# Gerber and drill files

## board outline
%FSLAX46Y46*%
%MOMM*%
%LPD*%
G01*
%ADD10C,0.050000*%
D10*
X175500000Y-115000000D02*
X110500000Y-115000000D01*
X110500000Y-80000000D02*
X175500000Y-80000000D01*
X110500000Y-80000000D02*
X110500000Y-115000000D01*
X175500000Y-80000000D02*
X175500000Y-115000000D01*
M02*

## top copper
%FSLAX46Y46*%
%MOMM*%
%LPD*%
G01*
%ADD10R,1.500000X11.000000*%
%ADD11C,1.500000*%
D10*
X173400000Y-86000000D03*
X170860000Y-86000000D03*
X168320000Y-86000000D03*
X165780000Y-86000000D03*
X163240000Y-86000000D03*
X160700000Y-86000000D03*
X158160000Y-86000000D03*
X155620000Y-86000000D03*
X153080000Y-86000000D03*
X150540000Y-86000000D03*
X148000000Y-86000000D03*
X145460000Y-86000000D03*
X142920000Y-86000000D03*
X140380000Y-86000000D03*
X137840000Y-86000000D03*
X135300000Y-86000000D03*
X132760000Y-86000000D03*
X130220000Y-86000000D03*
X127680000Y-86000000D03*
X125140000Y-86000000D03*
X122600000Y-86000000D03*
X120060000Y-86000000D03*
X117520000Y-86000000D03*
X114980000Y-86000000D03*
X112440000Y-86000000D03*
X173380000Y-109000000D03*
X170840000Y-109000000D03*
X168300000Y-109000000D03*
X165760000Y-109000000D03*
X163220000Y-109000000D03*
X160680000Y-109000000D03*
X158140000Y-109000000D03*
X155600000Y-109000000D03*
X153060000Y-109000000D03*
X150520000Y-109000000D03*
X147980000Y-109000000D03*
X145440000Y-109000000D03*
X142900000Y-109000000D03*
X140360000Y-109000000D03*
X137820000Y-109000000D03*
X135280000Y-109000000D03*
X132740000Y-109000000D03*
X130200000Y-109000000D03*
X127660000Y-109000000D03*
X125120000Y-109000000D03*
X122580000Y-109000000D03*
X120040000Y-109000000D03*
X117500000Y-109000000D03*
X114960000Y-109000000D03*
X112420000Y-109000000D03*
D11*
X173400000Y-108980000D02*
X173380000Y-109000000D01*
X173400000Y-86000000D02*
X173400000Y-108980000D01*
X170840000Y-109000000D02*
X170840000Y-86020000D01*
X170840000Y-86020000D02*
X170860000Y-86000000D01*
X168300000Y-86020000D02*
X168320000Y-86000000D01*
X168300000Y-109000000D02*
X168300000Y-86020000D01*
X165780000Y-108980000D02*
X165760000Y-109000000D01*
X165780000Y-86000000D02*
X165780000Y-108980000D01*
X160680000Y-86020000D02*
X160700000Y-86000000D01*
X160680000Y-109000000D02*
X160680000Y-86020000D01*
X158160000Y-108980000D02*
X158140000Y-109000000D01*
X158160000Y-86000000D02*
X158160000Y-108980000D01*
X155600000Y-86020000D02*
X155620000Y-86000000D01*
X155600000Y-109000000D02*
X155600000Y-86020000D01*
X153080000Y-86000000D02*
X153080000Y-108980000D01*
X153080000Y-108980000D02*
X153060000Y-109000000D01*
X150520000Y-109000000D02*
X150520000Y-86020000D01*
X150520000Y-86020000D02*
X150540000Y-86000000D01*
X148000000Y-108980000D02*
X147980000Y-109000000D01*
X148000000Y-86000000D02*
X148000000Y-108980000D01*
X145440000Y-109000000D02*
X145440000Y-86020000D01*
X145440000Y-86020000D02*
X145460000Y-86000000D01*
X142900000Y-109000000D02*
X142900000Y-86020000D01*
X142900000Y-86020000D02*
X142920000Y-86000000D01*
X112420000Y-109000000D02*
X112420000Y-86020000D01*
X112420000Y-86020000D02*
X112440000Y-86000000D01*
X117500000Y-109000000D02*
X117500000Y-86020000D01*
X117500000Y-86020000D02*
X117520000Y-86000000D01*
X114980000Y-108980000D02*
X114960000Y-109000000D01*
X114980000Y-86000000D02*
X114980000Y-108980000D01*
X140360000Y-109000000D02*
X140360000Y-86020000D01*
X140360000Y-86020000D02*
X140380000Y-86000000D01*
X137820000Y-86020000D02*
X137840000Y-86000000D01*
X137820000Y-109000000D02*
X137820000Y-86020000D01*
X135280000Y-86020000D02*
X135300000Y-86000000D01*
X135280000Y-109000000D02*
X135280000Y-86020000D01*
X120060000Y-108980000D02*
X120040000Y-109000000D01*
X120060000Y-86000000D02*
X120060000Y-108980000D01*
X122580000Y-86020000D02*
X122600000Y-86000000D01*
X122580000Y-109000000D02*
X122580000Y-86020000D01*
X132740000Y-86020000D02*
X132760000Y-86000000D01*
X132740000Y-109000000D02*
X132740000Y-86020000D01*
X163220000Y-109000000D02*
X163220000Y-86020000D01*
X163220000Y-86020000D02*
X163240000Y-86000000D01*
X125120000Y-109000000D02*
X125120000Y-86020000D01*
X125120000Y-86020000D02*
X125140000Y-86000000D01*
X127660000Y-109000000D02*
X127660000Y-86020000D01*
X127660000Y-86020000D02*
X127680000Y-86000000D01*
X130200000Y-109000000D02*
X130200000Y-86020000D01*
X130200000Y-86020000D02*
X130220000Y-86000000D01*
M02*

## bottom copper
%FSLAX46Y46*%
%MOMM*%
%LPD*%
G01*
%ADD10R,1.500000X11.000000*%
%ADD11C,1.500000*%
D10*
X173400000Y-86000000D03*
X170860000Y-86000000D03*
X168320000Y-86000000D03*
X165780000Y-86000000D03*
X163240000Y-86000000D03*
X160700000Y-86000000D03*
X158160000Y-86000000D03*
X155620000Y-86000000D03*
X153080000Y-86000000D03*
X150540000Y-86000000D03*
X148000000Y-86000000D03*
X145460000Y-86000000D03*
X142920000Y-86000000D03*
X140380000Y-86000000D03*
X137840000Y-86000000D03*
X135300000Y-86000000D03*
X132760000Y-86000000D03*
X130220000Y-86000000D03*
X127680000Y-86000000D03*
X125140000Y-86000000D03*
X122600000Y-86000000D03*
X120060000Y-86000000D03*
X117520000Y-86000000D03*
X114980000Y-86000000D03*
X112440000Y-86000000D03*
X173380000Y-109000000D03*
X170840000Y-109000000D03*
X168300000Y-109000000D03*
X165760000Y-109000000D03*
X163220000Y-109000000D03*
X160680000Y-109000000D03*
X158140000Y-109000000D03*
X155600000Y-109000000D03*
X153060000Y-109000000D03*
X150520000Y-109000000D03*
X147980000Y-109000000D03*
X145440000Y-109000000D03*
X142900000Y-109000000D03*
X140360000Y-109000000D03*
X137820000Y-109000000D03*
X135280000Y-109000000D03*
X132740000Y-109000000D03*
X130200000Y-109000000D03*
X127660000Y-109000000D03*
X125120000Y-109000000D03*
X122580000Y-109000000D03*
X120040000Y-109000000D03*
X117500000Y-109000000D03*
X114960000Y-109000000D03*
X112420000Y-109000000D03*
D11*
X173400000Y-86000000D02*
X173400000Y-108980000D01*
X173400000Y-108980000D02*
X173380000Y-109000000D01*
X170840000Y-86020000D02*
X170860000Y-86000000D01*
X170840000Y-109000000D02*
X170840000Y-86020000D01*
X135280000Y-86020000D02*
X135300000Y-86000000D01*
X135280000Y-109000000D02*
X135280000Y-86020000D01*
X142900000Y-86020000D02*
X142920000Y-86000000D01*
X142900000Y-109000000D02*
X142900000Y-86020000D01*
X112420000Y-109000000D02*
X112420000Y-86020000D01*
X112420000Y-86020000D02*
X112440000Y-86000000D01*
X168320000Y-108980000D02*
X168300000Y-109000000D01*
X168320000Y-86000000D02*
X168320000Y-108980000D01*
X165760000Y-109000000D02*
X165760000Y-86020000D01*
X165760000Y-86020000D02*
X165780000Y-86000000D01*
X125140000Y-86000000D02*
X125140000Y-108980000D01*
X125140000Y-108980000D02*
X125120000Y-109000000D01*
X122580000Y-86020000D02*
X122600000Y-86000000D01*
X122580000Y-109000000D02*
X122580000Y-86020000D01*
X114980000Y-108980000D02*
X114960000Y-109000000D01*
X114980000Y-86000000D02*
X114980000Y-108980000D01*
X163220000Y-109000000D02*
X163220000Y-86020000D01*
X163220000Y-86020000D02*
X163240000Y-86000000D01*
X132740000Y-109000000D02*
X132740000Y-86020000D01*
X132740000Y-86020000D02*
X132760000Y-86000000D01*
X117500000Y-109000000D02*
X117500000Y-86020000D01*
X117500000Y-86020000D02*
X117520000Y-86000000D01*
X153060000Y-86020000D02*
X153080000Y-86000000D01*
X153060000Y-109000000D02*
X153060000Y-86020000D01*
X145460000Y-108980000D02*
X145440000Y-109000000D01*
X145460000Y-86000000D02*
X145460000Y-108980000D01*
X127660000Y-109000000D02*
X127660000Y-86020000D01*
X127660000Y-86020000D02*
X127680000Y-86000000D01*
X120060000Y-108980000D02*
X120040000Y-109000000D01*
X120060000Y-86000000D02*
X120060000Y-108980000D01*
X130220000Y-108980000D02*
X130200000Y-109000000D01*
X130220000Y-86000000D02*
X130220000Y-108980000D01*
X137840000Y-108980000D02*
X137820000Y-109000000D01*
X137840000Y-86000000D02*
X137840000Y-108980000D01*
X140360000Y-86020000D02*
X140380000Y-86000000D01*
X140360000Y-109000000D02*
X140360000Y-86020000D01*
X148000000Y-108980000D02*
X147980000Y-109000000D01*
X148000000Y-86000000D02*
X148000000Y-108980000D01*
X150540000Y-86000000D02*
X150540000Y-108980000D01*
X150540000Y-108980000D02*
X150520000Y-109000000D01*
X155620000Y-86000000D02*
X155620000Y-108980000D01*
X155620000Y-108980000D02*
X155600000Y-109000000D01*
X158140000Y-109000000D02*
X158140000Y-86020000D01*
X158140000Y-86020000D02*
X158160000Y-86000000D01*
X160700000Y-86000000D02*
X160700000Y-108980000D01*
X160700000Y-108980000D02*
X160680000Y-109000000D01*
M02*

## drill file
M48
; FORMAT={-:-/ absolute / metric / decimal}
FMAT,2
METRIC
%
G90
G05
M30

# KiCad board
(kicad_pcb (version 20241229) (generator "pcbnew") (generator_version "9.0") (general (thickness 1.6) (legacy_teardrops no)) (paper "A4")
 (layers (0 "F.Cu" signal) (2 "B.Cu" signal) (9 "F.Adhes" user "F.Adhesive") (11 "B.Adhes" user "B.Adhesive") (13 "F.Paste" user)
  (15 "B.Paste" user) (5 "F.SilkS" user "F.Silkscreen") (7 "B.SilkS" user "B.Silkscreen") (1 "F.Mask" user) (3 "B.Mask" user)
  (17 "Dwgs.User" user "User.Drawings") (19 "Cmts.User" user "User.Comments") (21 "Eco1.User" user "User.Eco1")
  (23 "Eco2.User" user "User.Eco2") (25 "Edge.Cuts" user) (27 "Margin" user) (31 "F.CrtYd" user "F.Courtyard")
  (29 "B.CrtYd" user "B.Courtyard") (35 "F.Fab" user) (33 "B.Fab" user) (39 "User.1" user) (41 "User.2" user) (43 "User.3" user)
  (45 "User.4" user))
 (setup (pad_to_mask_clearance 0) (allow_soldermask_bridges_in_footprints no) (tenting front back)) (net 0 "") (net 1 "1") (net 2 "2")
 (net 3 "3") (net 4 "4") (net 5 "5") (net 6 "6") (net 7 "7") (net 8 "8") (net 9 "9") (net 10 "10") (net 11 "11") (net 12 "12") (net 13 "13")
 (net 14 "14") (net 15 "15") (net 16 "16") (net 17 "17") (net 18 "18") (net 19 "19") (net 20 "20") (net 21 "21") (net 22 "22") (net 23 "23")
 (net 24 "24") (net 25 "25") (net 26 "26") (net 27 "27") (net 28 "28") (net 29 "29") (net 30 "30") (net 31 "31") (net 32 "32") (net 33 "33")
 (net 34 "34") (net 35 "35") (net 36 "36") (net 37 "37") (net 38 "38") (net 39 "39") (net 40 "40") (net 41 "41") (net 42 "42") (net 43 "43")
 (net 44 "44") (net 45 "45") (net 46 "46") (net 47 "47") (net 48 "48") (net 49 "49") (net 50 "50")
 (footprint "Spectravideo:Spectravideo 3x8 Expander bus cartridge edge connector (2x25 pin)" (layer "F.Cu") (at 143 86)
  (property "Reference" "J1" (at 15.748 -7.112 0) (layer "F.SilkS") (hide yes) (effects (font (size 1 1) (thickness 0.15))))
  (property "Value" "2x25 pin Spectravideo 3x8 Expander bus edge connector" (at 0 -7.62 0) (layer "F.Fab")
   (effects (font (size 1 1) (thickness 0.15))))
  (pad "1" connect rect (at 30.4 0) (size 1.5 11) (layers "F.Cu" "F.Mask") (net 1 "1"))
  (pad "2" connect rect (at 30.4 0) (size 1.5 11) (layers "B.Cu" "B.Mask") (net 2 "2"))
  (pad "3" connect rect (at 27.86 0) (size 1.5 11) (layers "F.Cu" "F.Mask") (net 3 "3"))
  (pad "4" connect rect (at 27.86 0) (size 1.5 11) (layers "B.Cu" "B.Mask") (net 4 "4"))
  (pad "5" connect rect (at 25.32 0) (size 1.5 11) (layers "F.Cu" "F.Mask") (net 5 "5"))
  (pad "6" connect rect (at 25.32 0) (size 1.5 11) (layers "B.Cu" "B.Mask") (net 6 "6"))
  (pad "7" connect rect (at 22.78 0) (size 1.5 11) (layers "F.Cu" "F.Mask") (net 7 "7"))
  (pad "8" connect rect (at 22.78 0) (size 1.5 11) (layers "B.Cu" "B.Mask") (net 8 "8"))
  (pad "9" connect rect (at 20.24 0) (size 1.5 11) (layers "F.Cu" "F.Mask") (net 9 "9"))
  (pad "10" connect rect (at 20.24 0) (size 1.5 11) (layers "B.Cu" "B.Mask") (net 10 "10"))
  (pad "11" connect rect (at 17.7 0) (size 1.5 11) (layers "F.Cu" "F.Mask") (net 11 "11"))
  (pad "12" connect rect (at 17.7 0) (size 1.5 11) (layers "B.Cu" "B.Mask") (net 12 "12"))
  (pad "13" connect rect (at 15.16 0) (size 1.5 11) (layers "F.Cu" "F.Mask") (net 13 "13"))
  (pad "14" connect rect (at 15.16 0) (size 1.5 11) (layers "B.Cu" "B.Mask") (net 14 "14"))
  (pad "15" connect rect (at 12.62 0) (size 1.5 11) (layers "F.Cu" "F.Mask") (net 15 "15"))
  (pad "16" connect rect (at 12.62 0) (size 1.5 11) (layers "B.Cu" "B.Mask") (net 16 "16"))
  (pad "17" connect rect (at 10.08 0) (size 1.5 11) (layers "F.Cu" "F.Mask") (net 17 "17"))
  (pad "18" connect rect (at 10.08 0) (size 1.5 11) (layers "B.Cu" "B.Mask") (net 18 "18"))
  (pad "19" connect rect (at 7.54 0) (size 1.5 11) (layers "F.Cu" "F.Mask") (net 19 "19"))
  (pad "20" connect rect (at 7.54 0) (size 1.5 11) (layers "B.Cu" "B.Mask") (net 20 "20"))
  (pad "21" connect rect (at 5 0) (size 1.5 11) (layers "F.Cu" "F.Mask") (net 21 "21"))
  (pad "22" connect rect (at 5 0) (size 1.5 11) (layers "B.Cu" "B.Mask") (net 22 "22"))
  (pad "23" connect rect (at 2.46 0) (size 1.5 11) (layers "F.Cu" "F.Mask") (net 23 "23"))
  (pad "24" connect rect (at 2.46 0) (size 1.5 11) (layers "B.Cu" "B.Mask") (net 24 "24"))
  (pad "25" connect rect (at -0.08 0) (size 1.5 11) (layers "F.Cu" "F.Mask") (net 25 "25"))
  (pad "26" connect rect (at -0.08 0) (size 1.5 11) (layers "B.Cu" "B.Mask") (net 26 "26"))
  (pad "27" connect rect (at -2.62 0) (size 1.5 11) (layers "F.Cu" "F.Mask") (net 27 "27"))
  (pad "28" connect rect (at -2.62 0) (size 1.5 11) (layers "B.Cu" "B.Mask") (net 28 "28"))
  (pad "29" connect rect (at -5.16 0) (size 1.5 11) (layers "F.Cu" "F.Mask") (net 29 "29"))
  (pad "30" connect rect (at -5.16 0) (size 1.5 11) (layers "B.Cu" "B.Mask") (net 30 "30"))
  (pad "31" connect rect (at -7.7 0) (size 1.5 11) (layers "F.Cu" "F.Mask") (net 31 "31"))
  (pad "32" connect rect (at -7.7 0) (size 1.5 11) (layers "B.Cu" "B.Mask") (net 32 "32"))
  (pad "33" connect rect (at -10.24 0) (size 1.5 11) (layers "F.Cu" "F.Mask") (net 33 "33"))
  (pad "34" connect rect (at -10.24 0) (size 1.5 11) (layers "B.Cu" "B.Mask") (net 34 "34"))
  (pad "35" connect rect (at -12.78 0) (size 1.5 11) (layers "F.Cu" "F.Mask") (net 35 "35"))
  (pad "36" connect rect (at -12.78 0) (size 1.5 11) (layers "B.Cu" "B.Mask") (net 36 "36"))
  (pad "37" connect rect (at -15.32 0) (size 1.5 11) (layers "F.Cu" "F.Mask") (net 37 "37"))
  (pad "38" connect rect (at -15.32 0) (size 1.5 11) (layers "B.Cu" "B.Mask") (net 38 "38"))
  (pad "39" connect rect (at -17.86 0) (size 1.5 11) (layers "F.Cu" "F.Mask") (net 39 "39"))
  (pad "40" connect rect (at -17.86 0) (size 1.5 11) (layers "B.Cu" "B.Mask") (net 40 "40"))
  (pad "41" connect rect (at -20.4 0) (size 1.5 11) (layers "F.Cu" "F.Mask") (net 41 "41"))
  (pad "42" connect rect (at -20.4 0) (size 1.5 11) (layers "B.Cu" "B.Mask") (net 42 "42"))
  (pad "43" connect rect (at -22.94 0) (size 1.5 11) (layers "F.Cu" "F.Mask") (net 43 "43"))
  (pad "44" connect rect (at -22.94 0) (size 1.5 11) (layers "B.Cu" "B.Mask") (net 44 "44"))
  (pad "45" connect rect (at -25.48 0) (size 1.5 11) (layers "F.Cu" "F.Mask") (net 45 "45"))
  (pad "46" connect rect (at -25.48 0) (size 1.5 11) (layers "B.Cu" "B.Mask") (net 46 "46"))
  (pad "47" connect rect (at -28.02 0) (size 1.5 11) (layers "F.Cu" "F.Mask") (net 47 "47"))
  (pad "48" connect rect (at -28.02 0) (size 1.5 11) (layers "B.Cu" "B.Mask") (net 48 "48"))
  (pad "49" connect rect (at -30.56 0) (size 1.5 11) (layers "F.Cu" "F.Mask") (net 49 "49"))
  (pad "50" connect rect (at -30.56 0) (size 1.5 11) (layers "B.Cu" "B.Mask") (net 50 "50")))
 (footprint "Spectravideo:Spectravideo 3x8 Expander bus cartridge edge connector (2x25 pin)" (layer "F.Cu") (at 142.98 109)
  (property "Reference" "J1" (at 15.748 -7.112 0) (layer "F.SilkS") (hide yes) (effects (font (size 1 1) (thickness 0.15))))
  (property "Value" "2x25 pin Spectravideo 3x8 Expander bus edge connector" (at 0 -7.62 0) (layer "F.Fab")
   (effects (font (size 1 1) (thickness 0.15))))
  (pad "1" connect rect (at 30.4 0) (size 1.5 11) (layers "F.Cu" "F.Mask") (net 1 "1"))
  (pad "2" connect rect (at 30.4 0) (size 1.5 11) (layers "B.Cu" "B.Mask") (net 2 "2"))
  (pad "3" connect rect (at 27.86 0) (size 1.5 11) (layers "F.Cu" "F.Mask") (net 3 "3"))
  (pad "4" connect rect (at 27.86 0) (size 1.5 11) (layers "B.Cu" "B.Mask") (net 4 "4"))
  (pad "5" connect rect (at 25.32 0) (size 1.5 11) (layers "F.Cu" "F.Mask") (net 5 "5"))
  (pad "6" connect rect (at 25.32 0) (size 1.5 11) (layers "B.Cu" "B.Mask") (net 6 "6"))
  (pad "7" connect rect (at 22.78 0) (size 1.5 11) (layers "F.Cu" "F.Mask") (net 7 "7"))
  (pad "8" connect rect (at 22.78 0) (size 1.5 11) (layers "B.Cu" "B.Mask") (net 8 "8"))
  (pad "9" connect rect (at 20.24 0) (size 1.5 11) (layers "F.Cu" "F.Mask") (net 9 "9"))
  (pad "10" connect rect (at 20.24 0) (size 1.5 11) (layers "B.Cu" "B.Mask") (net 10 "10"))
  (pad "11" connect rect (at 17.7 0) (size 1.5 11) (layers "F.Cu" "F.Mask") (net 11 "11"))
  (pad "12" connect rect (at 17.7 0) (size 1.5 11) (layers "B.Cu" "B.Mask") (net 12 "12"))
  (pad "13" connect rect (at 15.16 0) (size 1.5 11) (layers "F.Cu" "F.Mask") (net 13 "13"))
  (pad "14" connect rect (at 15.16 0) (size 1.5 11) (layers "B.Cu" "B.Mask") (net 14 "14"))
  (pad "15" connect rect (at 12.62 0) (size 1.5 11) (layers "F.Cu" "F.Mask") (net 15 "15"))
  (pad "16" connect rect (at 12.62 0) (size 1.5 11) (layers "B.Cu" "B.Mask") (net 16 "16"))
  (pad "17" connect rect (at 10.08 0) (size 1.5 11) (layers "F.Cu" "F.Mask") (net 17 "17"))
  (pad "18" connect rect (at 10.08 0) (size 1.5 11) (layers "B.Cu" "B.Mask") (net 18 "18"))
  (pad "19" connect rect (at 7.54 0) (size 1.5 11) (layers "F.Cu" "F.Mask") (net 19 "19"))
  (pad "20" connect rect (at 7.54 0) (size 1.5 11) (layers "B.Cu" "B.Mask") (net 20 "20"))
  (pad "21" connect rect (at 5 0) (size 1.5 11) (layers "F.Cu" "F.Mask") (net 21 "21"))
  (pad "22" connect rect (at 5 0) (size 1.5 11) (layers "B.Cu" "B.Mask") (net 22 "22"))
  (pad "23" connect rect (at 2.46 0) (size 1.5 11) (layers "F.Cu" "F.Mask") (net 23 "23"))
  (pad "24" connect rect (at 2.46 0) (size 1.5 11) (layers "B.Cu" "B.Mask") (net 24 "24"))
  (pad "25" connect rect (at -0.08 0) (size 1.5 11) (layers "F.Cu" "F.Mask") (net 25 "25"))
  (pad "26" connect rect (at -0.08 0) (size 1.5 11) (layers "B.Cu" "B.Mask") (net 26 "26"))
  (pad "27" connect rect (at -2.62 0) (size 1.5 11) (layers "F.Cu" "F.Mask") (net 27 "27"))
  (pad "28" connect rect (at -2.62 0) (size 1.5 11) (layers "B.Cu" "B.Mask") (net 28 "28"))
  (pad "29" connect rect (at -5.16 0) (size 1.5 11) (layers "F.Cu" "F.Mask") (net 29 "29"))
  (pad "30" connect rect (at -5.16 0) (size 1.5 11) (layers "B.Cu" "B.Mask") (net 30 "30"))
  (pad "31" connect rect (at -7.7 0) (size 1.5 11) (layers "F.Cu" "F.Mask") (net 31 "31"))
  (pad "32" connect rect (at -7.7 0) (size 1.5 11) (layers "B.Cu" "B.Mask") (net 32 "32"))
  (pad "33" connect rect (at -10.24 0) (size 1.5 11) (layers "F.Cu" "F.Mask") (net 33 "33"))
  (pad "34" connect rect (at -10.24 0) (size 1.5 11) (layers "B.Cu" "B.Mask") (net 34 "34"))
  (pad "35" connect rect (at -12.78 0) (size 1.5 11) (layers "F.Cu" "F.Mask") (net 35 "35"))
  (pad "36" connect rect (at -12.78 0) (size 1.5 11) (layers "B.Cu" "B.Mask") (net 36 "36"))
  (pad "37" connect rect (at -15.32 0) (size 1.5 11) (layers "F.Cu" "F.Mask") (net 37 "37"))
  (pad "38" connect rect (at -15.32 0) (size 1.5 11) (layers "B.Cu" "B.Mask") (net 38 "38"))
  (pad "39" connect rect (at -17.86 0) (size 1.5 11) (layers "F.Cu" "F.Mask") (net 39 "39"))
  (pad "40" connect rect (at -17.86 0) (size 1.5 11) (layers "B.Cu" "B.Mask") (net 40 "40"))
  (pad "41" connect rect (at -20.4 0) (size 1.5 11) (layers "F.Cu" "F.Mask") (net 41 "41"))
  (pad "42" connect rect (at -20.4 0) (size 1.5 11) (layers "B.Cu" "B.Mask") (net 42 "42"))
  (pad "43" connect rect (at -22.94 0) (size 1.5 11) (layers "F.Cu" "F.Mask") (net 43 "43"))
  (pad "44" connect rect (at -22.94 0) (size 1.5 11) (layers "B.Cu" "B.Mask") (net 44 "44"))
  (pad "45" connect rect (at -25.48 0) (size 1.5 11) (layers "F.Cu" "F.Mask") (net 45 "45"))
  (pad "46" connect rect (at -25.48 0) (size 1.5 11) (layers "B.Cu" "B.Mask") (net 46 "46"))
  (pad "47" connect rect (at -28.02 0) (size 1.5 11) (layers "F.Cu" "F.Mask") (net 47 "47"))
  (pad "48" connect rect (at -28.02 0) (size 1.5 11) (layers "B.Cu" "B.Mask") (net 48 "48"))
  (pad "49" connect rect (at -30.56 0) (size 1.5 11) (layers "F.Cu" "F.Mask") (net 49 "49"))
  (pad "50" connect rect (at -30.56 0) (size 1.5 11) (layers "B.Cu" "B.Mask") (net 50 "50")))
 (gr_line (start 175.5 115) (end 110.5 115) (stroke (width 0.05) (type default)) (layer "Edge.Cuts"))
 (gr_line (start 110.5 80) (end 175.5 80) (stroke (width 0.05) (type default)) (layer "Edge.Cuts"))
 (gr_line (start 110.5 80) (end 110.5 115) (stroke (width 0.05) (type default)) (layer "Edge.Cuts"))
 (gr_line (start 175.5 80) (end 175.5 115) (stroke (width 0.05) (type default)) (layer "Edge.Cuts"))
 (segment (start 173.4 108.98) (end 173.38 109) (width 1.5) (layer "F.Cu") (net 1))
 (segment (start 173.4 86) (end 173.4 108.98) (width 1.5) (layer "F.Cu") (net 1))
 (segment (start 170.84 109) (end 170.84 86.02) (width 1.5) (layer "F.Cu") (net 3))
 (segment (start 170.84 86.02) (end 170.86 86) (width 1.5) (layer "F.Cu") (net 3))
 (segment (start 168.3 86.02) (end 168.32 86) (width 1.5) (layer "F.Cu") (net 5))
 (segment (start 168.3 109) (end 168.3 86.02) (width 1.5) (layer "F.Cu") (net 5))
 (segment (start 165.78 108.98) (end 165.76 109) (width 1.5) (layer "F.Cu") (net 7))
 (segment (start 165.78 86) (end 165.78 108.98) (width 1.5) (layer "F.Cu") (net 7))
 (segment (start 160.68 86.02) (end 160.7 86) (width 1.5) (layer "F.Cu") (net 11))
 (segment (start 160.68 109) (end 160.68 86.02) (width 1.5) (layer "F.Cu") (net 11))
 (segment (start 158.16 108.98) (end 158.14 109) (width 1.5) (layer "F.Cu") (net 13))
 (segment (start 158.16 86) (end 158.16 108.98) (width 1.5) (layer "F.Cu") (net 13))
 (segment (start 155.6 86.02) (end 155.62 86) (width 1.5) (layer "F.Cu") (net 15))
 (segment (start 155.6 109) (end 155.6 86.02) (width 1.5) (layer "F.Cu") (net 15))
 (segment (start 153.08 86) (end 153.08 108.98) (width 1.5) (layer "F.Cu") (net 17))
 (segment (start 153.08 108.98) (end 153.06 109) (width 1.5) (layer "F.Cu") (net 17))
 (segment (start 150.52 109) (end 150.52 86.02) (width 1.5) (layer "F.Cu") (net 19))
 (segment (start 150.52 86.02) (end 150.54 86) (width 1.5) (layer "F.Cu") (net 19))
 (segment (start 148 108.98) (end 147.98 109) (width 1.5) (layer "F.Cu") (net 21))
 (segment (start 148 86) (end 148 108.98) (width 1.5) (layer "F.Cu") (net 21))
 (segment (start 145.44 109) (end 145.44 86.02) (width 1.5) (layer "F.Cu") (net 23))
 (segment (start 145.44 86.02) (end 145.46 86) (width 1.5) (layer "F.Cu") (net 23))
 (segment (start 142.9 109) (end 142.9 86.02) (width 1.5) (layer "F.Cu") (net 25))
 (segment (start 142.9 86.02) (end 142.92 86) (width 1.5) (layer "F.Cu") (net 25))
 (segment (start 112.42 109) (end 112.42 86.02) (width 1.5) (layer "F.Cu") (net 49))
 (segment (start 112.42 86.02) (end 112.44 86) (width 1.5) (layer "F.Cu") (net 49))
 (segment (start 117.5 109) (end 117.5 86.02) (width 1.5) (layer "F.Cu") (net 45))
 (segment (start 117.5 86.02) (end 117.52 86) (width 1.5) (layer "F.Cu") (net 45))
 (segment (start 114.98 108.98) (end 114.96 109) (width 1.5) (layer "F.Cu") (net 47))
 (segment (start 114.98 86) (end 114.98 108.98) (width 1.5) (layer "F.Cu") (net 47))
 (segment (start 140.36 109) (end 140.36 86.02) (width 1.5) (layer "F.Cu") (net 27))
 (segment (start 140.36 86.02) (end 140.38 86) (width 1.5) (layer "F.Cu") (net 27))
 (segment (start 137.82 86.02) (end 137.84 86) (width 1.5) (layer "F.Cu") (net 29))
 (segment (start 137.82 109) (end 137.82 86.02) (width 1.5) (layer "F.Cu") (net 29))
 (segment (start 135.28 86.02) (end 135.3 86) (width 1.5) (layer "F.Cu") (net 31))
 (segment (start 135.28 109) (end 135.28 86.02) (width 1.5) (layer "F.Cu") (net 31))
 (segment (start 120.06 108.98) (end 120.04 109) (width 1.5) (layer "F.Cu") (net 43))
 (segment (start 120.06 86) (end 120.06 108.98) (width 1.5) (layer "F.Cu") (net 43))
 (segment (start 122.58 86.02) (end 122.6 86) (width 1.5) (layer "F.Cu") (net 41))
 (segment (start 122.58 109) (end 122.58 86.02) (width 1.5) (layer "F.Cu") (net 41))
 (segment (start 132.74 86.02) (end 132.76 86) (width 1.5) (layer "F.Cu") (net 33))
 (segment (start 132.74 109) (end 132.74 86.02) (width 1.5) (layer "F.Cu") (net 33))
 (segment (start 163.22 109) (end 163.22 86.02) (width 1.5) (layer "F.Cu") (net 9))
 (segment (start 163.22 86.02) (end 163.24 86) (width 1.5) (layer "F.Cu") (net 9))
 (segment (start 125.12 109) (end 125.12 86.02) (width 1.5) (layer "F.Cu") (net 39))
 (segment (start 125.12 86.02) (end 125.14 86) (width 1.5) (layer "F.Cu") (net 39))
 (segment (start 127.66 109) (end 127.66 86.02) (width 1.5) (layer "F.Cu") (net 37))
 (segment (start 127.66 86.02) (end 127.68 86) (width 1.5) (layer "F.Cu") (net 37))
 (segment (start 130.2 109) (end 130.2 86.02) (width 1.5) (layer "F.Cu") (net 35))
 (segment (start 130.2 86.02) (end 130.22 86) (width 1.5) (layer "F.Cu") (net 35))
 (segment (start 173.4 86) (end 173.4 108.98) (width 1.5) (layer "B.Cu") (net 2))
 (segment (start 173.4 108.98) (end 173.38 109) (width 1.5) (layer "B.Cu") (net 2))
 (segment (start 170.84 86.02) (end 170.86 86) (width 1.5) (layer "B.Cu") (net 4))
 (segment (start 170.84 109) (end 170.84 86.02) (width 1.5) (layer "B.Cu") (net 4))
 (segment (start 135.28 86.02) (end 135.3 86) (width 1.5) (layer "B.Cu") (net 32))
 (segment (start 135.28 109) (end 135.28 86.02) (width 1.5) (layer "B.Cu") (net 32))
 (segment (start 142.9 86.02) (end 142.92 86) (width 1.5) (layer "B.Cu") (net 26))
 (segment (start 142.9 109) (end 142.9 86.02) (width 1.5) (layer "B.Cu") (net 26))
 (segment (start 112.42 109) (end 112.42 86.02) (width 1.5) (layer "B.Cu") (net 50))
 (segment (start 112.42 86.02) (end 112.44 86) (width 1.5) (layer "B.Cu") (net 50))
 (segment (start 168.32 108.98) (end 168.3 109) (width 1.5) (layer "B.Cu") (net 6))
 (segment (start 168.32 86) (end 168.32 108.98) (width 1.5) (layer "B.Cu") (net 6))
 (segment (start 165.76 109) (end 165.76 86.02) (width 1.5) (layer "B.Cu") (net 8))
 (segment (start 165.76 86.02) (end 165.78 86) (width 1.5) (layer "B.Cu") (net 8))
 (segment (start 125.14 86) (end 125.14 108.98) (width 1.5) (layer "B.Cu") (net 40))
 (segment (start 125.14 108.98) (end 125.12 109) (width 1.5) (layer "B.Cu") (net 40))
 (segment (start 122.58 86.02) (end 122.6 86) (width 1.5) (layer "B.Cu") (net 42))
 (segment (start 122.58 109) (end 122.58 86.02) (width 1.5) (layer "B.Cu") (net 42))
 (segment (start 114.98 108.98) (end 114.96 109) (width 1.5) (layer "B.Cu") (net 48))
 (segment (start 114.98 86) (end 114.98 108.98) (width 1.5) (layer "B.Cu") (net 48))
 (segment (start 163.22 109) (end 163.22 86.02) (width 1.5) (layer "B.Cu") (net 10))
 (segment (start 163.22 86.02) (end 163.24 86) (width 1.5) (layer "B.Cu") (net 10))
 (segment (start 132.74 109) (end 132.74 86.02) (width 1.5) (layer "B.Cu") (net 34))
 (segment (start 132.74 86.02) (end 132.76 86) (width 1.5) (layer "B.Cu") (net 34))
 (segment (start 117.5 109) (end 117.5 86.02) (width 1.5) (layer "B.Cu") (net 46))
 (segment (start 117.5 86.02) (end 117.52 86) (width 1.5) (layer "B.Cu") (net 46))
 (segment (start 153.06 86.02) (end 153.08 86) (width 1.5) (layer "B.Cu") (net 18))
 (segment (start 153.06 109) (end 153.06 86.02) (width 1.5) (layer "B.Cu") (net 18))
 (segment (start 145.46 108.98) (end 145.44 109) (width 1.5) (layer "B.Cu") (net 24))
 (segment (start 145.46 86) (end 145.46 108.98) (width 1.5) (layer "B.Cu") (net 24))
 (segment (start 127.66 109) (end 127.66 86.02) (width 1.5) (layer "B.Cu") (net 38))
 (segment (start 127.66 86.02) (end 127.68 86) (width 1.5) (layer "B.Cu") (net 38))
 (segment (start 120.06 108.98) (end 120.04 109) (width 1.5) (layer "B.Cu") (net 44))
 (segment (start 120.06 86) (end 120.06 108.98) (width 1.5) (layer "B.Cu") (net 44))
 (segment (start 130.22 108.98) (end 130.2 109) (width 1.5) (layer "B.Cu") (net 36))
 (segment (start 130.22 86) (end 130.22 108.98) (width 1.5) (layer "B.Cu") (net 36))
 (segment (start 137.84 108.98) (end 137.82 109) (width 1.5) (layer "B.Cu") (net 30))
 (segment (start 137.84 86) (end 137.84 108.98) (width 1.5) (layer "B.Cu") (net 30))
 (segment (start 140.36 86.02) (end 140.38 86) (width 1.5) (layer "B.Cu") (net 28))
 (segment (start 140.36 109) (end 140.36 86.02) (width 1.5) (layer "B.Cu") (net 28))
 (segment (start 148 108.98) (end 147.98 109) (width 1.5) (layer "B.Cu") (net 22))
 (segment (start 148 86) (end 148 108.98) (width 1.5) (layer "B.Cu") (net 22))
 (segment (start 150.54 86) (end 150.54 108.98) (width 1.5) (layer "B.Cu") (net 20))
 (segment (start 150.54 108.98) (end 150.52 109) (width 1.5) (layer "B.Cu") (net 20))
 (segment (start 155.62 86) (end 155.62 108.98) (width 1.5) (layer "B.Cu") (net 16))
 (segment (start 155.62 108.98) (end 155.6 109) (width 1.5) (layer "B.Cu") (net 16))
 (segment (start 158.14 109) (end 158.14 86.02) (width 1.5) (layer "B.Cu") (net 14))
 (segment (start 158.14 86.02) (end 158.16 86) (width 1.5) (layer "B.Cu") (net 14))
 (segment (start 160.7 86) (end 160.7 108.98) (width 1.5) (layer "B.Cu") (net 12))
 (segment (start 160.7 108.98) (end 160.68 109) (width 1.5) (layer "B.Cu") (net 12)))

